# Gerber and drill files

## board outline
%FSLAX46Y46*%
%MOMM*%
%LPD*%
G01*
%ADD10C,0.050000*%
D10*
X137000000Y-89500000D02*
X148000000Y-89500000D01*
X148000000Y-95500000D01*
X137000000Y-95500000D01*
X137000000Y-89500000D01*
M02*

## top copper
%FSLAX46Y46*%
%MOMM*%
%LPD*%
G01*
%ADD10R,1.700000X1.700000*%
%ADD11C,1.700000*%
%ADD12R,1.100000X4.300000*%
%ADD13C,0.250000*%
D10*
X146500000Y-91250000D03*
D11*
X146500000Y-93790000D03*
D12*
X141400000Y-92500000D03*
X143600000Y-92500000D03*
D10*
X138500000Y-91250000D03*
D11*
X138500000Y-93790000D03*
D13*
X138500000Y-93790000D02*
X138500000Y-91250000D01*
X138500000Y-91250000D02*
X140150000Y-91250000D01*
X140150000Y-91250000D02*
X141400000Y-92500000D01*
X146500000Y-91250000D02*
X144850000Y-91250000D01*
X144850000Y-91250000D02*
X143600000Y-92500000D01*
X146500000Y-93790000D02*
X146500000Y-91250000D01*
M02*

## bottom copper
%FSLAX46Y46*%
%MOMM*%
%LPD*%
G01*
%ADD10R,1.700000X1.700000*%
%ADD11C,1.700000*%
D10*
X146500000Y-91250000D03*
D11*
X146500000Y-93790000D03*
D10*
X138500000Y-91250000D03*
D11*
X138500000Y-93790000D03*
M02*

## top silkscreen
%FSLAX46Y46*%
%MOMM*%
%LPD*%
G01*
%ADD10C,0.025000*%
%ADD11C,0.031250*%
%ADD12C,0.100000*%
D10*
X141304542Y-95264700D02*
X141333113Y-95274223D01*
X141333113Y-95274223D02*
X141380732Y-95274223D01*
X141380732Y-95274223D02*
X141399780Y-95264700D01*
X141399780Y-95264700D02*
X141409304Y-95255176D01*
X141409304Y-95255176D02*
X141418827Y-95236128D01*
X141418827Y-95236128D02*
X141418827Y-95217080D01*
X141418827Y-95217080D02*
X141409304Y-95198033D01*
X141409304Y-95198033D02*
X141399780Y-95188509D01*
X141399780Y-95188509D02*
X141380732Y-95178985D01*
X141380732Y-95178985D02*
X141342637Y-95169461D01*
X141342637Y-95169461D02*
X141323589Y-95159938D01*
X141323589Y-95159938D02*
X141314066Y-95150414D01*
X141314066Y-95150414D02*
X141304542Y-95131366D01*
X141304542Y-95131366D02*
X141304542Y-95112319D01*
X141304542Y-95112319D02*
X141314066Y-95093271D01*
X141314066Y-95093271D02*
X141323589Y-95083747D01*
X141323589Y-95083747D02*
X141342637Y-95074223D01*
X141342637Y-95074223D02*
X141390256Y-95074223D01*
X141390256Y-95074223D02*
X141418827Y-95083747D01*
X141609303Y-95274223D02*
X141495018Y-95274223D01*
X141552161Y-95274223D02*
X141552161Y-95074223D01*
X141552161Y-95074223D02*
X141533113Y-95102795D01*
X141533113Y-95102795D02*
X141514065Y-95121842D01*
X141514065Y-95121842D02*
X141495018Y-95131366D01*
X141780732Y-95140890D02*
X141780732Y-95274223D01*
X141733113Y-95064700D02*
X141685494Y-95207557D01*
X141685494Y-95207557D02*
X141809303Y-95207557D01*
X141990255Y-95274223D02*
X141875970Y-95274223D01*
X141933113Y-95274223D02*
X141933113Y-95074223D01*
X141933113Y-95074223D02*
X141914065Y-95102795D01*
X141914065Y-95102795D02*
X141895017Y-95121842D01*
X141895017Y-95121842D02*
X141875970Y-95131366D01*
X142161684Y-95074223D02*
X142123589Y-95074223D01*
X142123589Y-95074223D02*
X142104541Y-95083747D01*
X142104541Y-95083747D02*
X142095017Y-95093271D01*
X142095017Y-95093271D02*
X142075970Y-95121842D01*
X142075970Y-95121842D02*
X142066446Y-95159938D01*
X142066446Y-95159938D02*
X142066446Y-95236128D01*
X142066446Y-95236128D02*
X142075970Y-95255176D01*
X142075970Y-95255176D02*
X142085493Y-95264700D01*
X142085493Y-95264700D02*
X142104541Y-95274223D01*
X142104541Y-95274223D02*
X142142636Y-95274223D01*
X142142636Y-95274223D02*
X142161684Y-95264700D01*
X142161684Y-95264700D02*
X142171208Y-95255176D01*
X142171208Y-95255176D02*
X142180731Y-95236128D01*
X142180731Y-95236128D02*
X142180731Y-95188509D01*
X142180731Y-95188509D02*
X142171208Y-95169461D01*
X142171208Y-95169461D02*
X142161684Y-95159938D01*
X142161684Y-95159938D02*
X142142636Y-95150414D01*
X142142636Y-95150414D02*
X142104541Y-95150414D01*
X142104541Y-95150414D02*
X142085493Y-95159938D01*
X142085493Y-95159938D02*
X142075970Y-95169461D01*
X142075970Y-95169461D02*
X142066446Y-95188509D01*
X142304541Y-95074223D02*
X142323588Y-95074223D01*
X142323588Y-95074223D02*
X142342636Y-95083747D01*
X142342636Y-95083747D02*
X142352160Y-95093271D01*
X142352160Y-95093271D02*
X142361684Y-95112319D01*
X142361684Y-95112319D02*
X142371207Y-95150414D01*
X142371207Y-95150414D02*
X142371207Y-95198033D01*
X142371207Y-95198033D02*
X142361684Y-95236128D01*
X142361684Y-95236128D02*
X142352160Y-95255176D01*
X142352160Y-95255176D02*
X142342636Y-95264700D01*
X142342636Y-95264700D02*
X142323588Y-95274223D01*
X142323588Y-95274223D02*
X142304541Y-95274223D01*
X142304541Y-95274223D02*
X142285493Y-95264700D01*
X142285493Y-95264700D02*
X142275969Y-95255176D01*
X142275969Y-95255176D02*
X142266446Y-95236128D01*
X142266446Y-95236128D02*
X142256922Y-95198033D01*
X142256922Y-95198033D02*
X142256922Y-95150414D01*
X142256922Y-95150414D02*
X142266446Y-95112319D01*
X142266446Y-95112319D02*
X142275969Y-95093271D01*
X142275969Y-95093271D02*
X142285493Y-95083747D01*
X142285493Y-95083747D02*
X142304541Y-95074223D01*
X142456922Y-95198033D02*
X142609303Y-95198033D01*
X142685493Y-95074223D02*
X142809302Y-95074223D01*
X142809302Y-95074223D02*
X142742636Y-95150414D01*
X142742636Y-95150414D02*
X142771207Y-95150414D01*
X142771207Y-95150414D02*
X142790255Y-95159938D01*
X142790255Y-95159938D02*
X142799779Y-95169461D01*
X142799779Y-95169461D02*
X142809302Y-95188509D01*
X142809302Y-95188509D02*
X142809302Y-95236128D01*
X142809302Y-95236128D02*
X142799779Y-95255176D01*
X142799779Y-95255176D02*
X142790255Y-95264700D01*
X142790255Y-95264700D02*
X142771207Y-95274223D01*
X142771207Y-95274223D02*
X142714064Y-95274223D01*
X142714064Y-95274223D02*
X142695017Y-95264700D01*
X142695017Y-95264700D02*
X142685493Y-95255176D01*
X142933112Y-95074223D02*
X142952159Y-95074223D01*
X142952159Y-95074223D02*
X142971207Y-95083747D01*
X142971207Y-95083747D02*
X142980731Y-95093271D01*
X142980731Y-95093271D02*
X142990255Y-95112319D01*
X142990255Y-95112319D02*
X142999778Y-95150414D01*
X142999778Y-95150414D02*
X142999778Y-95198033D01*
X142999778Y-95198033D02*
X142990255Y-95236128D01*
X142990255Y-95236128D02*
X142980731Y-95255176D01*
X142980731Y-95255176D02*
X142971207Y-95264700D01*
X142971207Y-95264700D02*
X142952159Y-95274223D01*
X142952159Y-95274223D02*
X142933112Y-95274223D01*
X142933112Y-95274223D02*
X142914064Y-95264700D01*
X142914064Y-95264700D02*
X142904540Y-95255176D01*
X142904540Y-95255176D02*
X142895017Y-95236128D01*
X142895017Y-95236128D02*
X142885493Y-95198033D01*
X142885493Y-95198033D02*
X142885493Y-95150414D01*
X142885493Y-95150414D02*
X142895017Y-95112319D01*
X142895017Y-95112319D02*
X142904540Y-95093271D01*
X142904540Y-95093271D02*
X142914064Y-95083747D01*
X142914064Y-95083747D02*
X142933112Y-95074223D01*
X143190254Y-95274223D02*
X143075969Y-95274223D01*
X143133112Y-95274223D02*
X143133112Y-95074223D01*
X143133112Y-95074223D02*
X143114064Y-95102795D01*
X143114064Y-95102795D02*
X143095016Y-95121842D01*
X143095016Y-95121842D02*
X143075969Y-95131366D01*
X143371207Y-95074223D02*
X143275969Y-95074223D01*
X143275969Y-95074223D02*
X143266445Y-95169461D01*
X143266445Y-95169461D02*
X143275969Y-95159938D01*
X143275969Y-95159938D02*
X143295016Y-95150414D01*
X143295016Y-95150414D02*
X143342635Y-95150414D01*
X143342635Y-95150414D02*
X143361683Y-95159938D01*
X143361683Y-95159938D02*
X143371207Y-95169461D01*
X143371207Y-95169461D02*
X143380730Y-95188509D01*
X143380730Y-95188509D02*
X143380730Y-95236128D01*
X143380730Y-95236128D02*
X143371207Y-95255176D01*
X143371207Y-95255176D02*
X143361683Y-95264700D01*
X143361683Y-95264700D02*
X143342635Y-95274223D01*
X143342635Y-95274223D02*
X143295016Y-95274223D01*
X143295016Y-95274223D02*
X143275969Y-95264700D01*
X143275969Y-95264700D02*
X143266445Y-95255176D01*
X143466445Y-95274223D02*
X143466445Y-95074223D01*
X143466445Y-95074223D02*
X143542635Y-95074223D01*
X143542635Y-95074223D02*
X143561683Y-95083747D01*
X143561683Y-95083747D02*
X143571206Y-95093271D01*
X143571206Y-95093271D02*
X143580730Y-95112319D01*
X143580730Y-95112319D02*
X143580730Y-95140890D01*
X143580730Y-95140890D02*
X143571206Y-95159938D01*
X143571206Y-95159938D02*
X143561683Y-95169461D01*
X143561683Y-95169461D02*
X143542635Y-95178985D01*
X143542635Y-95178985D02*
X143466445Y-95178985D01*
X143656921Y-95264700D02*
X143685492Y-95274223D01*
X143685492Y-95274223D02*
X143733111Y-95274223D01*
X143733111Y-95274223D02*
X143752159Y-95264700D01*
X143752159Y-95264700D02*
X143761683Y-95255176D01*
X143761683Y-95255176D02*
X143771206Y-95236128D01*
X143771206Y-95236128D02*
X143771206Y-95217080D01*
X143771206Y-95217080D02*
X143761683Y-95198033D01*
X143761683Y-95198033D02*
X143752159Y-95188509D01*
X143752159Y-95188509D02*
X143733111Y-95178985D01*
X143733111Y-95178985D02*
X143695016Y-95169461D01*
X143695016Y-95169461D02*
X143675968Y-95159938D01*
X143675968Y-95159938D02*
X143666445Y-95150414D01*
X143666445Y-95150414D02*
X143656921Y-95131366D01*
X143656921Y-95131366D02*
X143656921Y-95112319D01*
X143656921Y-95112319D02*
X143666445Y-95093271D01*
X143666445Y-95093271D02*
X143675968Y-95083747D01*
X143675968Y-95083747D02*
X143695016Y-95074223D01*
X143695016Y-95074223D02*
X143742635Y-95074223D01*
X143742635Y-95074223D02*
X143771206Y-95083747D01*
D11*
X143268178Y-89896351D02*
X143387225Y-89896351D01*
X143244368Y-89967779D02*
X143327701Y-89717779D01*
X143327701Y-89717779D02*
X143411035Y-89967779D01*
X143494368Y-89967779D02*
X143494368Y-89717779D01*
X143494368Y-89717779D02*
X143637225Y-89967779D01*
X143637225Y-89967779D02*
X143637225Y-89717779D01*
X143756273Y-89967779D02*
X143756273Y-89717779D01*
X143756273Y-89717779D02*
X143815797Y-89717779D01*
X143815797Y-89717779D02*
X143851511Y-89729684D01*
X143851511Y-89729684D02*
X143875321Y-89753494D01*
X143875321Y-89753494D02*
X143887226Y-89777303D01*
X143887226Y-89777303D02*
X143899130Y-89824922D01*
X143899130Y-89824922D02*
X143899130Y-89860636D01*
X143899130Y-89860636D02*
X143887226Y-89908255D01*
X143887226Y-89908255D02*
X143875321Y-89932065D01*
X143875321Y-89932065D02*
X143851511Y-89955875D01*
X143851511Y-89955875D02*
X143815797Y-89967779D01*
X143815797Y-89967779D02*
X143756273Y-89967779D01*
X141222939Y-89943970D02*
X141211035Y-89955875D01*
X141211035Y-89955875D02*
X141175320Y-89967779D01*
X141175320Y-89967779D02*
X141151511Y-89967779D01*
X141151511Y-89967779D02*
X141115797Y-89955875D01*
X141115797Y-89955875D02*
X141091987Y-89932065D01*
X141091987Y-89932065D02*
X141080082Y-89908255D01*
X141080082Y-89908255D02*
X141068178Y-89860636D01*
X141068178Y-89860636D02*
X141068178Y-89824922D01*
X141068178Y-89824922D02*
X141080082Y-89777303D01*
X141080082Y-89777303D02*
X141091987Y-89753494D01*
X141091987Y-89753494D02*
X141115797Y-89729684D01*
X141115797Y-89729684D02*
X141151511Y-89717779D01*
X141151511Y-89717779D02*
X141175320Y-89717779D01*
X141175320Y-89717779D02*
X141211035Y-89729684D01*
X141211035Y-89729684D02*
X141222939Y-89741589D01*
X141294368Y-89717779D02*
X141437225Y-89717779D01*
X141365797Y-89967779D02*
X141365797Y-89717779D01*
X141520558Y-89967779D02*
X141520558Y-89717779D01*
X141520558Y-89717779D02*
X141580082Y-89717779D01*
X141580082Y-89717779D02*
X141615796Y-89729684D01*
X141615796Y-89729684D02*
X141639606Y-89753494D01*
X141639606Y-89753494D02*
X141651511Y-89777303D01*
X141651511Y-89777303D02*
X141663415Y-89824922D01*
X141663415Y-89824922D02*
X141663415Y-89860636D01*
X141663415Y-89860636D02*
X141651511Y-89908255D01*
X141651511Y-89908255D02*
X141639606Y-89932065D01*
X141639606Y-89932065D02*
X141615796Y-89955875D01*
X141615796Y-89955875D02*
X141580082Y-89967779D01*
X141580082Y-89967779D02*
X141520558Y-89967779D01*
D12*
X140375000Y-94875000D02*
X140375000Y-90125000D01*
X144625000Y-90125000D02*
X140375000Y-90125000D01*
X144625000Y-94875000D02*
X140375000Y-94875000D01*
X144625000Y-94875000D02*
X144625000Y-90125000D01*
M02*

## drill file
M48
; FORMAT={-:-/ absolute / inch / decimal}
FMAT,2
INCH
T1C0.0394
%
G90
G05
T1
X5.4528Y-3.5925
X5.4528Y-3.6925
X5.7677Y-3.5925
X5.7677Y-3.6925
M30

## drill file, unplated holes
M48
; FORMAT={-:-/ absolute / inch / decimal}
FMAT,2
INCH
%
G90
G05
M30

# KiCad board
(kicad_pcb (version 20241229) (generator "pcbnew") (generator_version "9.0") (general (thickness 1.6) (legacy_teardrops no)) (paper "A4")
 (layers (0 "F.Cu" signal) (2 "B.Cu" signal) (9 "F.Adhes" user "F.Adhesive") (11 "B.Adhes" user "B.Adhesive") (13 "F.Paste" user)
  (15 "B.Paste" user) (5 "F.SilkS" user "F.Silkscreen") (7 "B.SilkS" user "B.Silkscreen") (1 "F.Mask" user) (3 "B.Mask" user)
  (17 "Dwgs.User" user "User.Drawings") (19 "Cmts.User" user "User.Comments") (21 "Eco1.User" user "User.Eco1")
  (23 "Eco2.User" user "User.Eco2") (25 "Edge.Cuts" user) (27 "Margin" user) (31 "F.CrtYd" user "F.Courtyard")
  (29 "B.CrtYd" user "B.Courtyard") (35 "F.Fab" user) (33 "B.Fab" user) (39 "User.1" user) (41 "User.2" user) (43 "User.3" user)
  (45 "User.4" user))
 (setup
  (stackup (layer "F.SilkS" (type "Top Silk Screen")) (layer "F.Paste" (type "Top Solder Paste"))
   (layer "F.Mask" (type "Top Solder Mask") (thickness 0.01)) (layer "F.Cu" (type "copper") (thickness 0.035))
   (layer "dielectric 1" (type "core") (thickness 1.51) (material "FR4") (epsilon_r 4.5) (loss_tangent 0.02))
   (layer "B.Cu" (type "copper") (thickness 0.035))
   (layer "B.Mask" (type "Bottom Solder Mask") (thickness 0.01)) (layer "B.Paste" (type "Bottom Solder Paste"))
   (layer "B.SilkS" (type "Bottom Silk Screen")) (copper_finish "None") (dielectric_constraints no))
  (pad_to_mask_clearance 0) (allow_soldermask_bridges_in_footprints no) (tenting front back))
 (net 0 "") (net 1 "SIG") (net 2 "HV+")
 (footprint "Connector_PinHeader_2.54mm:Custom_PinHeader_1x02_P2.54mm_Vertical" (layer "F.Cu") (at 146.5 91.25)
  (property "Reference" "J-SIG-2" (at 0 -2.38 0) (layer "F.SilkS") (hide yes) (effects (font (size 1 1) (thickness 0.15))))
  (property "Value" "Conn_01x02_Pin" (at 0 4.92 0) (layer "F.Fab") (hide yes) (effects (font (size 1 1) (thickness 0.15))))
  (pad "1" thru_hole rect (at 0 0) (size 1.7 1.7) (drill 1) (layers "*.Cu" "*.Mask") (remove_unused_layers no) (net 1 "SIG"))
  (pad "2" thru_hole circle (at 0 2.54) (size 1.7 1.7) (drill 1) (layers "*.Cu" "*.Mask") (remove_unused_layers no) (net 1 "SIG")))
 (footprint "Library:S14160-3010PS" (layer "F.Cu") (at 142.5 92.5)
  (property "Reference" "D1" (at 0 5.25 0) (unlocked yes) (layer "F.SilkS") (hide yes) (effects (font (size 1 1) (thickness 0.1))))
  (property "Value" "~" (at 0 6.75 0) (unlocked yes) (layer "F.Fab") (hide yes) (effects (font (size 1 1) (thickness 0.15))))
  (fp_line (start -2.125 2.375) (end -2.125 -2.375) (stroke (width 0.1) (type default)) (layer "F.SilkS"))
  (fp_line (start 2.125 -2.375) (end -2.125 -2.375) (stroke (width 0.1) (type default)) (layer "F.SilkS"))
  (fp_line (start 2.125 2.375) (end -2.125 2.375) (stroke (width 0.1) (type default)) (layer "F.SilkS"))
  (fp_line (start 2.125 2.375) (end 2.125 -2.375) (stroke (width 0.1) (type default)) (layer "F.SilkS"))
  (pad "1" smd rect (at -1.1 0) (size 1.1 4.3) (layers "F.Cu" "F.Mask" "F.Paste") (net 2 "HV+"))
  (pad "2" smd rect (at 1.1 0) (size 1.1 4.3) (layers "F.Cu" "F.Mask" "F.Paste") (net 1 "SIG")))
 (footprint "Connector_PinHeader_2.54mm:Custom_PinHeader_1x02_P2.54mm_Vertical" (layer "F.Cu") (at 138.5 91.25)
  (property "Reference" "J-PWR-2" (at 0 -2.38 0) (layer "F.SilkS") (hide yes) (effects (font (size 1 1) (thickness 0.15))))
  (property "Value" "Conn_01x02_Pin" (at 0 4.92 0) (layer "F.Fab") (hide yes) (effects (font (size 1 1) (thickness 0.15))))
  (pad "1" thru_hole rect (at 0 0) (size 1.7 1.7) (drill 1) (layers "*.Cu" "*.Mask") (remove_unused_layers no) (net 2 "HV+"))
  (pad "2" thru_hole circle (at 0 2.54) (size 1.7 1.7) (drill 1) (layers "*.Cu" "*.Mask") (remove_unused_layers no) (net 2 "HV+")))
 (gr_rect (start 137 89.5) (end 148 95.5) (stroke (width 0.05) (type default)) (fill no) (layer "Edge.Cuts"))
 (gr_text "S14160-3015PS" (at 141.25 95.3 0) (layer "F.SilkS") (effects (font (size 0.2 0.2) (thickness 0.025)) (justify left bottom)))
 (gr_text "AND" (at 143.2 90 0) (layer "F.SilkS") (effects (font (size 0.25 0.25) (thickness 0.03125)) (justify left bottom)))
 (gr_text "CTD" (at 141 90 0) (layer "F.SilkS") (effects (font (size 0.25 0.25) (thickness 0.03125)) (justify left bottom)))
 (segment (start 138.5 93.79) (end 138.5 91.25) (width 0.25) (layer "F.Cu") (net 2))
 (segment (start 138.5 91.25) (end 140.15 91.25) (width 0.25) (layer "F.Cu") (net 2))
 (segment (start 140.15 91.25) (end 141.4 92.5) (width 0.25) (layer "F.Cu") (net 2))
 (segment (start 146.5 91.25) (end 144.85 91.25) (width 0.25) (layer "F.Cu") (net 1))
 (segment (start 144.85 91.25) (end 143.6 92.5) (width 0.25) (layer "F.Cu") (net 1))
 (segment (start 146.5 93.79) (end 146.5 91.25) (width 0.25) (layer "F.Cu") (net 1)))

